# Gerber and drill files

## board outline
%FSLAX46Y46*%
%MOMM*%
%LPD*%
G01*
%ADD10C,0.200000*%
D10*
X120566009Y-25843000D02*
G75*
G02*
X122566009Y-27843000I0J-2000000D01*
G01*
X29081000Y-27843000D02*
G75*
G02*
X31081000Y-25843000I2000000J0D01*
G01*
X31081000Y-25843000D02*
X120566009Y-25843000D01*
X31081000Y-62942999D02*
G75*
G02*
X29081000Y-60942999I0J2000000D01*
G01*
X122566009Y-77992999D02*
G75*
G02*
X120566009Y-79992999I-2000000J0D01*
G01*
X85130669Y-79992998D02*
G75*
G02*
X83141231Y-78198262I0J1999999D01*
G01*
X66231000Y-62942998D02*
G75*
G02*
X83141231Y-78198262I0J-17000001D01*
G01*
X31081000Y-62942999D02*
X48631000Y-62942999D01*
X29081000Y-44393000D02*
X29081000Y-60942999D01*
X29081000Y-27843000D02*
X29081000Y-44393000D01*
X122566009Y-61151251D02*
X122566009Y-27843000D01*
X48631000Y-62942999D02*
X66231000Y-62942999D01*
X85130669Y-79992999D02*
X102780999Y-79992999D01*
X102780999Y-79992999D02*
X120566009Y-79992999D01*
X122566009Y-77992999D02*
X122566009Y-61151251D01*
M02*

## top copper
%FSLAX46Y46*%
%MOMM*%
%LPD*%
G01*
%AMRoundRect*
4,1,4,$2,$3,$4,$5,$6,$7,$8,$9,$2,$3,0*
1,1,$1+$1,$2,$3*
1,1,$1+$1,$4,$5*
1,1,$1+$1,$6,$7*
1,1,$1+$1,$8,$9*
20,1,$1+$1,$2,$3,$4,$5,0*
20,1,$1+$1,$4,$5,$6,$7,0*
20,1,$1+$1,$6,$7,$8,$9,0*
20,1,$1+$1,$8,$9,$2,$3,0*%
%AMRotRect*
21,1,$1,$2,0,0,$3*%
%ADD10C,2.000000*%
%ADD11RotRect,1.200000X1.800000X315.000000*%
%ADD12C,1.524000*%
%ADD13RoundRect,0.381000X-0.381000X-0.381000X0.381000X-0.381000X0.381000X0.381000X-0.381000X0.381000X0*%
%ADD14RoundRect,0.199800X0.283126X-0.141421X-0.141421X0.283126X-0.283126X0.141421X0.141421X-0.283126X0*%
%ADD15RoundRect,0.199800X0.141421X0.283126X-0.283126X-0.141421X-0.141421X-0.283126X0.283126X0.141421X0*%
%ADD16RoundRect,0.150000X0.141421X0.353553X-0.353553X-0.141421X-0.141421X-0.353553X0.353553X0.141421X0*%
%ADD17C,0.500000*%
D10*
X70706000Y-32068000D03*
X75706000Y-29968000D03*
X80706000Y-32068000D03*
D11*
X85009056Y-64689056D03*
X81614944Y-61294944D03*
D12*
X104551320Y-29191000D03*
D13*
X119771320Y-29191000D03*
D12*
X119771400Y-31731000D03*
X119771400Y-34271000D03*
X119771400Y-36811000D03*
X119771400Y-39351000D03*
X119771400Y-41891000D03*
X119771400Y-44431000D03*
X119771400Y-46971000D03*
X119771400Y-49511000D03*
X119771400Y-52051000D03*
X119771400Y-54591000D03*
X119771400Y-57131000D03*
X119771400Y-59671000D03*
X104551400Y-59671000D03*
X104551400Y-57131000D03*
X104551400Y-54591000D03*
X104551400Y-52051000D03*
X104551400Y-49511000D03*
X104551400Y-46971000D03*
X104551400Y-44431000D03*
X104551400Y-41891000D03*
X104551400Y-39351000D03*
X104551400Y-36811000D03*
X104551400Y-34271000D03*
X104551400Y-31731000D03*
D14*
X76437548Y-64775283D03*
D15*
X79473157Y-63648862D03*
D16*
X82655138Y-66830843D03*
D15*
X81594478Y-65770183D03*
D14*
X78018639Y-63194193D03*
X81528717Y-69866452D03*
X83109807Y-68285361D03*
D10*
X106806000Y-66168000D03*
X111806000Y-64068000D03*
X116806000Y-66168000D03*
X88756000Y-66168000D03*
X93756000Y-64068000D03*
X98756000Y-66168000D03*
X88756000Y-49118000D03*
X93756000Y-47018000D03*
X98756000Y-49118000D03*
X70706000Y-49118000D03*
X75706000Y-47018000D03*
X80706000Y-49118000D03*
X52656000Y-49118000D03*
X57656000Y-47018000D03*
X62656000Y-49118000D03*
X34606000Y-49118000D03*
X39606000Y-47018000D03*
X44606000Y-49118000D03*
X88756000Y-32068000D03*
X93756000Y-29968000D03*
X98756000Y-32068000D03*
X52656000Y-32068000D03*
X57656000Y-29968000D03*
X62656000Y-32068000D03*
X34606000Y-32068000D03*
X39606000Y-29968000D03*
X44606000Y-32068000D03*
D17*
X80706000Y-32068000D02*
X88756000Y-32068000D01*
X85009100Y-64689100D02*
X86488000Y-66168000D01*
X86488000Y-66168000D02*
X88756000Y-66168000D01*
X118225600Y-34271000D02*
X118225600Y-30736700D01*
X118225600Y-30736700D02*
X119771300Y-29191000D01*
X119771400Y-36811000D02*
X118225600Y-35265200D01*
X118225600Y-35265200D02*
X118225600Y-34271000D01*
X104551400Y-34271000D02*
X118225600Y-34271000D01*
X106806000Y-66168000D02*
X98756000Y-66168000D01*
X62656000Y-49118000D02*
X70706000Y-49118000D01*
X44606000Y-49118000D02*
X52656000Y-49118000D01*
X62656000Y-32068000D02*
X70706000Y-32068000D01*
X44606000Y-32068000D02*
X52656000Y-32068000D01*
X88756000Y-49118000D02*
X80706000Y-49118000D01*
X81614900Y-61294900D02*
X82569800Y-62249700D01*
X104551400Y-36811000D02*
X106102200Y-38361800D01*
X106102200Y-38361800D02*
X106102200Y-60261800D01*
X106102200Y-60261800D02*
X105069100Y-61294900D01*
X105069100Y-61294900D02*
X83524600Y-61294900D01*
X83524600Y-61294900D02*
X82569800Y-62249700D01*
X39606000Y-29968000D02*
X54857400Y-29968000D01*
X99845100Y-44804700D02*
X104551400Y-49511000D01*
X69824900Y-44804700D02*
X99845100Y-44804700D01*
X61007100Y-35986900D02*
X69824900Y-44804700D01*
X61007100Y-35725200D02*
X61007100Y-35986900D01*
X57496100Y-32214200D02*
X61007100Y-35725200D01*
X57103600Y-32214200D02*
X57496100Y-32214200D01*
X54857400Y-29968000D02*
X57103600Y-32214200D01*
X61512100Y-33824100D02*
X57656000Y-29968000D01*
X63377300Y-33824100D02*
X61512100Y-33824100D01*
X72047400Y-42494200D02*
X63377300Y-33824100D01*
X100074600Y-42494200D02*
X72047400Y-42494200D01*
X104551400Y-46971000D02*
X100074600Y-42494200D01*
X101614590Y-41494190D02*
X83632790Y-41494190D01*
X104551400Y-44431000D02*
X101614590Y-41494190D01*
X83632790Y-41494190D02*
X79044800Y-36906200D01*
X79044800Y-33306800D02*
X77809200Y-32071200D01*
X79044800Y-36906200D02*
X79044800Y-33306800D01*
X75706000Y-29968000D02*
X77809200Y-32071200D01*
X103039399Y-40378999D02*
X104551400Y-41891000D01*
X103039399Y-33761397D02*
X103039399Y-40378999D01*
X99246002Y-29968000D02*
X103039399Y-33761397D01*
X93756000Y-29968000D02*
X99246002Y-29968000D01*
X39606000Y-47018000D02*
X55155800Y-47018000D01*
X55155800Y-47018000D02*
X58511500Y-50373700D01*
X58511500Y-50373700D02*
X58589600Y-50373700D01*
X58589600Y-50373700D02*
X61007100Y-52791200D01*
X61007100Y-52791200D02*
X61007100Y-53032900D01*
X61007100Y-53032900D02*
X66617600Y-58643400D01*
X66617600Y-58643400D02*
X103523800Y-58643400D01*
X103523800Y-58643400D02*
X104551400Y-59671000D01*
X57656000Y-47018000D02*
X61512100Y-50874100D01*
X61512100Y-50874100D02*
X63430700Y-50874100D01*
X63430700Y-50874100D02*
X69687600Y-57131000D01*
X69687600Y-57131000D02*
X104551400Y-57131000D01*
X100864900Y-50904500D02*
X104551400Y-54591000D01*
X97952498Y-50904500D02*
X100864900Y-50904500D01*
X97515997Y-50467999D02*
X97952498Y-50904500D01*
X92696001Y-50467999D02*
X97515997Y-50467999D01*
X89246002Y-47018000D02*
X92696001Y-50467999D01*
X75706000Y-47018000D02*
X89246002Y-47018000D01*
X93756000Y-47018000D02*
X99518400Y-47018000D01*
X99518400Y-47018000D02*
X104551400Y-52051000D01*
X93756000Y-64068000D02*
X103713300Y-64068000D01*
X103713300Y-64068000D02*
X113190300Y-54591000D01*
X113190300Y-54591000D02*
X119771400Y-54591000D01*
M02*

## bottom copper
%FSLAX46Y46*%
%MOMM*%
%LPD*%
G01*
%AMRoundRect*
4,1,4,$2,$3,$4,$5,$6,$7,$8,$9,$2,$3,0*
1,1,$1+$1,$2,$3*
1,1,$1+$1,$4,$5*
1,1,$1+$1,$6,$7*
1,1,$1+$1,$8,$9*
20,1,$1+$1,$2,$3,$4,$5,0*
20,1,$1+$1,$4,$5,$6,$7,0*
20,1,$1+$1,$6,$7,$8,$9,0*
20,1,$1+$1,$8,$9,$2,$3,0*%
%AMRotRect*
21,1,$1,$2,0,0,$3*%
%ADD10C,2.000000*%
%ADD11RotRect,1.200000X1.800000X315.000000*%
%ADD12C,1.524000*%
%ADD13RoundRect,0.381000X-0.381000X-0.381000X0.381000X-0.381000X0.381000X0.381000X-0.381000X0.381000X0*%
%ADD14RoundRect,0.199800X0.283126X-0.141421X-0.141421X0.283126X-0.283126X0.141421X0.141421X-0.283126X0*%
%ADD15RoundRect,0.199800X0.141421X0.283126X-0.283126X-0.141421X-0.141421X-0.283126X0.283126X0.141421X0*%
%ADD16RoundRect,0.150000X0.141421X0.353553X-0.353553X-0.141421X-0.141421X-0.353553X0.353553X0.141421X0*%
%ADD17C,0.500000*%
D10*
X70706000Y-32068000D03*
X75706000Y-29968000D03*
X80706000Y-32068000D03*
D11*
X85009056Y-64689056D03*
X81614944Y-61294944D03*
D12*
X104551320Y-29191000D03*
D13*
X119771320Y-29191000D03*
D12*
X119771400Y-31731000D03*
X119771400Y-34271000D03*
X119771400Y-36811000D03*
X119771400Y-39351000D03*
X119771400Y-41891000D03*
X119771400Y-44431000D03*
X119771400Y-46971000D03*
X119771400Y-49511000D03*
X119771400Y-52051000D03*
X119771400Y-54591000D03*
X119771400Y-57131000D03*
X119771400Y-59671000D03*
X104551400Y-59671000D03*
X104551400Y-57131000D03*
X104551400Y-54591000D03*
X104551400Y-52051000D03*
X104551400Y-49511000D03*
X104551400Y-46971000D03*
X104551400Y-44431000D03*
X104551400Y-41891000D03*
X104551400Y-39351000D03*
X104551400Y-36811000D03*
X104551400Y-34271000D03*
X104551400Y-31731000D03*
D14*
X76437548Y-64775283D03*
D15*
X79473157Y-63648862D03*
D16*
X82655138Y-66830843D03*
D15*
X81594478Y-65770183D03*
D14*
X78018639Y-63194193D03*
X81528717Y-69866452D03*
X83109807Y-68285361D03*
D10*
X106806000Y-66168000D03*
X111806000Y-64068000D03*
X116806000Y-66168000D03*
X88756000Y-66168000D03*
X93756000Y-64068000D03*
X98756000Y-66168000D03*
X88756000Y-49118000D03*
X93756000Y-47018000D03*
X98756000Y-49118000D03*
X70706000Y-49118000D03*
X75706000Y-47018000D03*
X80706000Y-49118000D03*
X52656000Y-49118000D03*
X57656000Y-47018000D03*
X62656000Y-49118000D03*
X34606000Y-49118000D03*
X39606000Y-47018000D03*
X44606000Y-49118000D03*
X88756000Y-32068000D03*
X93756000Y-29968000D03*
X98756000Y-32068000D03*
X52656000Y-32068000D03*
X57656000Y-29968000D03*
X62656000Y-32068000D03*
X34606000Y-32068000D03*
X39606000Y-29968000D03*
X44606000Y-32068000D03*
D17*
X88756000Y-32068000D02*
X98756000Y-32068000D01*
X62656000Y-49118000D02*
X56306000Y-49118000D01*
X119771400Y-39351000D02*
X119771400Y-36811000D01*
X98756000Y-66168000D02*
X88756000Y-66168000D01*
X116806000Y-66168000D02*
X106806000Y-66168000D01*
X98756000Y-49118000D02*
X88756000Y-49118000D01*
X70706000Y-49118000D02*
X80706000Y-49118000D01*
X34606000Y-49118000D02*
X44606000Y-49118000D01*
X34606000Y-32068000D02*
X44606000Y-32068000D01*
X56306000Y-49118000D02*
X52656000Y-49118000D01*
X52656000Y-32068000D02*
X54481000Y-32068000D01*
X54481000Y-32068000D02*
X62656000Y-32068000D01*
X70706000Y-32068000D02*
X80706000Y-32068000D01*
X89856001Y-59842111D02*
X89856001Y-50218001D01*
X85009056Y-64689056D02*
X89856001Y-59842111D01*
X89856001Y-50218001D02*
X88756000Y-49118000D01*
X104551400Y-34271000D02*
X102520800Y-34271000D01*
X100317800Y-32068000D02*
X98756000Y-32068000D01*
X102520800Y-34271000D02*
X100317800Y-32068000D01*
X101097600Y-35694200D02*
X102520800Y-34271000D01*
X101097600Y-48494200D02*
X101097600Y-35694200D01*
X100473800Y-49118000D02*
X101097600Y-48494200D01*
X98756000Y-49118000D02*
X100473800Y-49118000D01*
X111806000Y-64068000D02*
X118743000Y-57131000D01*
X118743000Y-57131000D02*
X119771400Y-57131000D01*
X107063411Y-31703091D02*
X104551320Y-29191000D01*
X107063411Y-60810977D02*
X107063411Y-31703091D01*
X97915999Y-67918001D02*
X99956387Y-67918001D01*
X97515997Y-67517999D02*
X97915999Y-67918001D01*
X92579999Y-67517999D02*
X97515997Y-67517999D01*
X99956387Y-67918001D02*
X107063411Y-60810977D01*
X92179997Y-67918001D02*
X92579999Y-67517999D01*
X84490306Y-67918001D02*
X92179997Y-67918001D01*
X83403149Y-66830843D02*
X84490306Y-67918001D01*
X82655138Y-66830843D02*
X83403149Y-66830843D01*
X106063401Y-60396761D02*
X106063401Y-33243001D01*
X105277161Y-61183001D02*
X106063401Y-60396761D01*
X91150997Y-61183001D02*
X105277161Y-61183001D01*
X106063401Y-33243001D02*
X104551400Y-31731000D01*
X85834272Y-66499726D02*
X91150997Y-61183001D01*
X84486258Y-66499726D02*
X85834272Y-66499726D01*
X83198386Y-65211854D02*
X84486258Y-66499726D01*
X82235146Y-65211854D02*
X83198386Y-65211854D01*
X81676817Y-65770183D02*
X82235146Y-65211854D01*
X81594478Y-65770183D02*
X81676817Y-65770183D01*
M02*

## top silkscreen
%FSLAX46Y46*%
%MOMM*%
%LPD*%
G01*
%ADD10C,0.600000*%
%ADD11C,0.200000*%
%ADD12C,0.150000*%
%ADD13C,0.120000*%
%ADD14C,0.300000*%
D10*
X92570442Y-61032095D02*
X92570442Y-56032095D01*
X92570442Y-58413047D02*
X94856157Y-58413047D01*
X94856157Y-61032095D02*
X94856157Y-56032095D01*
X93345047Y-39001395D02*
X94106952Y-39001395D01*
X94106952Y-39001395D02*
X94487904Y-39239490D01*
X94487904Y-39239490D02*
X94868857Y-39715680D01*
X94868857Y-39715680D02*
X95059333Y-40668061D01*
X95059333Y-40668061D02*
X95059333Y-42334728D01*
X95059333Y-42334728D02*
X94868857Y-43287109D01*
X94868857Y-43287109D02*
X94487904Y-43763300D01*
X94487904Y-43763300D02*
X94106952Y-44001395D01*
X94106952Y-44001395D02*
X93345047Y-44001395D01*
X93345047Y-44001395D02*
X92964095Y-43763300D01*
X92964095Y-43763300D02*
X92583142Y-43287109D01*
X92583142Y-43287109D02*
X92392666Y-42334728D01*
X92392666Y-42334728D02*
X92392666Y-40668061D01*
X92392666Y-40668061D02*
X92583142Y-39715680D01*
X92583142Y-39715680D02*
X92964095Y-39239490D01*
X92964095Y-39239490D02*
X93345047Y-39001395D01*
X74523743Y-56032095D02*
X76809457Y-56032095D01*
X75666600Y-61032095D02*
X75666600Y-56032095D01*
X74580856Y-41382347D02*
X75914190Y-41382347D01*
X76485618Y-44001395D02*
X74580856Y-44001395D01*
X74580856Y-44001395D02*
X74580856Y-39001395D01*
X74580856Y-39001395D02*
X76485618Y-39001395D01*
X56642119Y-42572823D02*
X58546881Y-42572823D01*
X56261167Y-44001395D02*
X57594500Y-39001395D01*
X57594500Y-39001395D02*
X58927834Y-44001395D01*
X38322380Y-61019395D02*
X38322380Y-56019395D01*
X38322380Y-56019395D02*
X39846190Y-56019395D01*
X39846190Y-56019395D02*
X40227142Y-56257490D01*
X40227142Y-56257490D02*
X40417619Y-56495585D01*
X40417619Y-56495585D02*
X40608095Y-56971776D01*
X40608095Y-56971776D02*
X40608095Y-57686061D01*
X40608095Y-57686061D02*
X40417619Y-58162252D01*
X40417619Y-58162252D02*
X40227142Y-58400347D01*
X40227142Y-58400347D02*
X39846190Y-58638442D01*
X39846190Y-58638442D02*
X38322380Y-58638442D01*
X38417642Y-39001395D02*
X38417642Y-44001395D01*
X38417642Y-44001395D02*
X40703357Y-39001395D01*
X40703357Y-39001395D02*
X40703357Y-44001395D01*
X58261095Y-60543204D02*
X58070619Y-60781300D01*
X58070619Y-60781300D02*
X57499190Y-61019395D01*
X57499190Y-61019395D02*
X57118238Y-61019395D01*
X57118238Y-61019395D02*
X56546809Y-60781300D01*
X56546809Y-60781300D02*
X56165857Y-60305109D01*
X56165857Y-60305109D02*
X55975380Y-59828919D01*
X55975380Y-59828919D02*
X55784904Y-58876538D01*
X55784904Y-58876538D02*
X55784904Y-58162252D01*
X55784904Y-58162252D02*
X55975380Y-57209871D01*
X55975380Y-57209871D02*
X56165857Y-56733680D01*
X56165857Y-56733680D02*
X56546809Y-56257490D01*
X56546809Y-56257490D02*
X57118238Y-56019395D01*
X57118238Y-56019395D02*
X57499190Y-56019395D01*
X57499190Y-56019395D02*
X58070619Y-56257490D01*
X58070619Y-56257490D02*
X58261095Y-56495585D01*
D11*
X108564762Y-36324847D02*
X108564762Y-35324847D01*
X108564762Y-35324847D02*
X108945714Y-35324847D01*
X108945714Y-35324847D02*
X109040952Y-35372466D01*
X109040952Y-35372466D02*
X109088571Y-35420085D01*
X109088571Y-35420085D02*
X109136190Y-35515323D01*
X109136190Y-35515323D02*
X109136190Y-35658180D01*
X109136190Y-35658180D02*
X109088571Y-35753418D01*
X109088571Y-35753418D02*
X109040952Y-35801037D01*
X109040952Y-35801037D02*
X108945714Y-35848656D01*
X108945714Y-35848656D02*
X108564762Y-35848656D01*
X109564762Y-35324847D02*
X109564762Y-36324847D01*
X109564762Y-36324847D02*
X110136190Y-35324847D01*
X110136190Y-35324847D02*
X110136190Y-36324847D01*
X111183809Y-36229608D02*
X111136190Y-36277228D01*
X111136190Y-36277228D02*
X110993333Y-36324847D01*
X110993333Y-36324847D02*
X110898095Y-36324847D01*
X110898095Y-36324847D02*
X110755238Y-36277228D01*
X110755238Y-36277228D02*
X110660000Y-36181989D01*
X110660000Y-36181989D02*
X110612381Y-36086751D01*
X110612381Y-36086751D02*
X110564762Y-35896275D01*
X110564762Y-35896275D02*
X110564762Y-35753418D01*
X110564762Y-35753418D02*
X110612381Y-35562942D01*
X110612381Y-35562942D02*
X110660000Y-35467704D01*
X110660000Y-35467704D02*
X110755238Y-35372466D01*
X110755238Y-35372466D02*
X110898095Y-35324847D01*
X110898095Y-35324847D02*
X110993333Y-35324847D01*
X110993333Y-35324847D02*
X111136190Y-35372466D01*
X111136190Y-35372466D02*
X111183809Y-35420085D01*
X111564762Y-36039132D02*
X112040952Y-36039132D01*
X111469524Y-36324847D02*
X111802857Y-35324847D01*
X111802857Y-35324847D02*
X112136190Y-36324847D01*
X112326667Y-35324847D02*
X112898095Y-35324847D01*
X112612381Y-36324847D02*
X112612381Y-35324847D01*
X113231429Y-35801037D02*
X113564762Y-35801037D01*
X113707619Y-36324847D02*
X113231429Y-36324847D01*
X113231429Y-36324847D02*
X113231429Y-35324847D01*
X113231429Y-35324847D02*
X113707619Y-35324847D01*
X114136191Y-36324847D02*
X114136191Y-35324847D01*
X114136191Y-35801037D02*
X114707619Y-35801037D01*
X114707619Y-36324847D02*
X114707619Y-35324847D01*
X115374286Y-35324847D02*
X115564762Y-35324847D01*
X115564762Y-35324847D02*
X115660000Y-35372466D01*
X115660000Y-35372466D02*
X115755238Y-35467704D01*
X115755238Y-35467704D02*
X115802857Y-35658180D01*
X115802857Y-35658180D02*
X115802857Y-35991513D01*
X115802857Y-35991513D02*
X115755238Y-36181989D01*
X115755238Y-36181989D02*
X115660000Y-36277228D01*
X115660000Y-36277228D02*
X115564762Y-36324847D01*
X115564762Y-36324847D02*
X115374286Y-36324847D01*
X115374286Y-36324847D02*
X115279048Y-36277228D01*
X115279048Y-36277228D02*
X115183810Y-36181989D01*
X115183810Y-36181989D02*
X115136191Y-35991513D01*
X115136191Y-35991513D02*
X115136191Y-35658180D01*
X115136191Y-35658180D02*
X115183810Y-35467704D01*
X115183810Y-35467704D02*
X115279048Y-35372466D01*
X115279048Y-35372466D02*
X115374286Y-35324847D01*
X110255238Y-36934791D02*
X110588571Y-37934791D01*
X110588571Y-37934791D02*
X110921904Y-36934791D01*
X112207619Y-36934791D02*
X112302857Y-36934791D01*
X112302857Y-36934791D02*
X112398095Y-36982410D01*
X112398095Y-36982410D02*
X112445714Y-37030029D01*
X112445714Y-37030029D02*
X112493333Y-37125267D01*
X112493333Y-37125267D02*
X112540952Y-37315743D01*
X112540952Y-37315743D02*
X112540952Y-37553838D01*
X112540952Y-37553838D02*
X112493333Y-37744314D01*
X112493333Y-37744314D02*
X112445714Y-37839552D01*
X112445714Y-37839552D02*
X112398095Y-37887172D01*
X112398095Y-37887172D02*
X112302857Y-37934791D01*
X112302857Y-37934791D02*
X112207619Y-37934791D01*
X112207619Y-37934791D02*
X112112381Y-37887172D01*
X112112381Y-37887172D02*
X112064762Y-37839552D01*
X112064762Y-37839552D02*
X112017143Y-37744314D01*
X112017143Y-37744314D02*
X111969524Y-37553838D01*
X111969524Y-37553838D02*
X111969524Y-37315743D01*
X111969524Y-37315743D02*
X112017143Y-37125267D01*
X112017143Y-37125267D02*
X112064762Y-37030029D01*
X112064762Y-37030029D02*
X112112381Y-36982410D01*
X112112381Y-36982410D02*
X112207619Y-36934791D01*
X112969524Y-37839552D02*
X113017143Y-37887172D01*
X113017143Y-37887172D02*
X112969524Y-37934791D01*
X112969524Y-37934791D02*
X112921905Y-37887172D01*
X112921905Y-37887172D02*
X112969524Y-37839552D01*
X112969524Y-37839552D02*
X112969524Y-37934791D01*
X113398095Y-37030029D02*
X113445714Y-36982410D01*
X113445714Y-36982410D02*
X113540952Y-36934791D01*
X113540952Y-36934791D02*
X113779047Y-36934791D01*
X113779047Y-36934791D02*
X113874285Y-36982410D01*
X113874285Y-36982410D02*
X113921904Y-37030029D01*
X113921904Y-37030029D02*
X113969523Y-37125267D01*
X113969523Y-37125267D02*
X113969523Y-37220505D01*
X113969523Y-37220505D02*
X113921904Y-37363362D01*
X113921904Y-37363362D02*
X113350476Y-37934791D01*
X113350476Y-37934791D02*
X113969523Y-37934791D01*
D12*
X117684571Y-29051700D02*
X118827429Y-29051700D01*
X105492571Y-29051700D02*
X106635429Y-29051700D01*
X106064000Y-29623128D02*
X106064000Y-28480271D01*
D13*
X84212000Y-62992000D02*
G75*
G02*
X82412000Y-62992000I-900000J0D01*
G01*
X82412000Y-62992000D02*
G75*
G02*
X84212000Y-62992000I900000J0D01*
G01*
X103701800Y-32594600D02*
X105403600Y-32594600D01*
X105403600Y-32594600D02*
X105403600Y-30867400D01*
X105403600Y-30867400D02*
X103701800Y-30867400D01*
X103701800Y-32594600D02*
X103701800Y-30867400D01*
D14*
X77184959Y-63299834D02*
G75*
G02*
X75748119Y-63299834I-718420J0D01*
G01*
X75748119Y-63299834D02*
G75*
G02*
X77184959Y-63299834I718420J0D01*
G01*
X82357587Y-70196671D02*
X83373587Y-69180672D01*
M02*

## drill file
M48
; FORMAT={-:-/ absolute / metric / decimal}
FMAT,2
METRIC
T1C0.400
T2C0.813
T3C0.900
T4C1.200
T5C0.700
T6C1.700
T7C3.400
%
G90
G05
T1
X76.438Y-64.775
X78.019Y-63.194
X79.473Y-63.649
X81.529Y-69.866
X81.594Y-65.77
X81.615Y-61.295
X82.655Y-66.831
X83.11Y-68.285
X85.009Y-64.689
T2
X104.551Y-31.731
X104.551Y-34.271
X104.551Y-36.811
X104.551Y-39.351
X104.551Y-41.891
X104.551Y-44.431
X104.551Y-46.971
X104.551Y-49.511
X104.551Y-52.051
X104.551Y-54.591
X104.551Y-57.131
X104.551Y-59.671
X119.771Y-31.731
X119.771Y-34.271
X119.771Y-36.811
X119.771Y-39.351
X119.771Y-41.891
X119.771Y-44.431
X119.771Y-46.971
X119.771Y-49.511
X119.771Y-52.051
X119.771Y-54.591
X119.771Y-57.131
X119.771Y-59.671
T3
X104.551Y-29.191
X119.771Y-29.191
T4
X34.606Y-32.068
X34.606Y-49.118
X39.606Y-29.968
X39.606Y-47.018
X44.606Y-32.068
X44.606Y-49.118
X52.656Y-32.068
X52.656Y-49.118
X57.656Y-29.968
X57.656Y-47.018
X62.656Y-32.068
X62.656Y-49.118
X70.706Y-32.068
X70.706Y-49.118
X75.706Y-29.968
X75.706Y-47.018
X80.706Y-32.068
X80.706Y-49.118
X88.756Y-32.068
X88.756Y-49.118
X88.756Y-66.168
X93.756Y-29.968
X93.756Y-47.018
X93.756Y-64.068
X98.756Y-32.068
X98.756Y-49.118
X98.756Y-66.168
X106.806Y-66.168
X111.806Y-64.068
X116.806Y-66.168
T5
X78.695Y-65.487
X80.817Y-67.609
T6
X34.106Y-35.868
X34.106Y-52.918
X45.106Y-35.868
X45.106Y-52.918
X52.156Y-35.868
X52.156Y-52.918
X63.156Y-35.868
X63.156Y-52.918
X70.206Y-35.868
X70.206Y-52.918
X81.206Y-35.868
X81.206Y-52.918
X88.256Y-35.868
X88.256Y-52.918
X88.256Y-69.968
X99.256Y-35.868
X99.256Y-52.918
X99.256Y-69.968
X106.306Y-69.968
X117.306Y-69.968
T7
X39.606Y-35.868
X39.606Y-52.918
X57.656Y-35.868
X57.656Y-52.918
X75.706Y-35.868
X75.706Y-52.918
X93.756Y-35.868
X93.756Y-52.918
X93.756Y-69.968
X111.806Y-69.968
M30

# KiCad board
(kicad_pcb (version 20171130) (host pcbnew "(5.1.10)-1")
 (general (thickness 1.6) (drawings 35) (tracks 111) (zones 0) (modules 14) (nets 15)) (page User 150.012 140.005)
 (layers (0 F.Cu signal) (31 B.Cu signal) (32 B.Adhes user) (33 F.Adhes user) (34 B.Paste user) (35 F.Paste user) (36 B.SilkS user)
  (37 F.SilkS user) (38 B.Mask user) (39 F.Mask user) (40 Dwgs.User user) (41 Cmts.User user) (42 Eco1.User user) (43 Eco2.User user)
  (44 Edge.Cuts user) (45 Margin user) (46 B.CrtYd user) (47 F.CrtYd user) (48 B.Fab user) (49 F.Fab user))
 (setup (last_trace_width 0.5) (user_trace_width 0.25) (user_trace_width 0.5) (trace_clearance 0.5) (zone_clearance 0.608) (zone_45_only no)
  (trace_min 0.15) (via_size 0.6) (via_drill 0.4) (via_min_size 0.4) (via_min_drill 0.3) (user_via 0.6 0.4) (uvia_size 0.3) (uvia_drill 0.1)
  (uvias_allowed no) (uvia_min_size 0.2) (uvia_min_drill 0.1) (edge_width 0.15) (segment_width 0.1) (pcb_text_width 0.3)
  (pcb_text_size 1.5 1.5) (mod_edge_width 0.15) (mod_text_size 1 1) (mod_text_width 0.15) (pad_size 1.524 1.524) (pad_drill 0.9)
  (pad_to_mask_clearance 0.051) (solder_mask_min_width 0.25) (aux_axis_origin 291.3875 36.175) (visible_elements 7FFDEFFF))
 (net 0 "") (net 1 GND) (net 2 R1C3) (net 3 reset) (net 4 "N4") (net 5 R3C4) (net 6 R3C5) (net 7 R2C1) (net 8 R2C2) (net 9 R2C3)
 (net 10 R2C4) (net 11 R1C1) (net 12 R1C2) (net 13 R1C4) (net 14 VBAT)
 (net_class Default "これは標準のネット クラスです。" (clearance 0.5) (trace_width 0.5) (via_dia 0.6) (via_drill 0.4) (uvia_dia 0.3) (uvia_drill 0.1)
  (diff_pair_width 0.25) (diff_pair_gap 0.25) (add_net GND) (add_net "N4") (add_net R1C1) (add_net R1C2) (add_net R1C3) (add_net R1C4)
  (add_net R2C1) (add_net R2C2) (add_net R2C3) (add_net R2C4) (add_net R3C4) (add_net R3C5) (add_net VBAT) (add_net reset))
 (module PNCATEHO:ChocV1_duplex (layer F.Cu) (at 75.706 35.868)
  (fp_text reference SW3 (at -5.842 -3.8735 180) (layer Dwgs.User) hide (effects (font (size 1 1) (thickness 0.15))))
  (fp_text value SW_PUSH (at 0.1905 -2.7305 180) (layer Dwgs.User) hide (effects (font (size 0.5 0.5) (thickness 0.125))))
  (pad 2 thru_hole circle (at -5 -3.8) (size 2 2) (drill 1.2) (layers *.Cu *.Mask) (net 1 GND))
  (pad 1 thru_hole circle (at 0 -5.9) (size 2 2) (drill 1.2) (layers *.Cu *.Mask) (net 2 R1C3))
  (pad "" np_thru_hole circle (at 5.5 0 90) (size 1.7 1.7) (drill 1.7) (layers *.Cu *.Mask))
  (pad "" np_thru_hole circle (at -5.5 0 90) (size 1.7 1.7) (drill 1.7) (layers *.Cu *.Mask))
  (pad "" np_thru_hole circle (at 0 0 90) (size 3.4 3.4) (drill 3.4) (layers *.Cu *.Mask))
  (pad 2 thru_hole circle (at 5 -3.8) (size 2 2) (drill 1.2) (layers *.Cu *.Mask) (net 1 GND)))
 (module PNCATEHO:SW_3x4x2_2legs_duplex (layer F.Cu) (at 83.312 62.992 315)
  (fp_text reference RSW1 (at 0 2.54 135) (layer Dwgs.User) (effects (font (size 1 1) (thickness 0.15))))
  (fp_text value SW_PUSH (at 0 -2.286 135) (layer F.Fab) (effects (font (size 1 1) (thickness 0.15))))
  (fp_circle (center 0 0) (end 0.9 0) (layer F.SilkS) (width 0.12))
  (pad 2 thru_hole rect (at 2.4 0 315) (size 1.2 1.8) (drill 0.4) (layers *.Cu *.Mask) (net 1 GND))
  (pad 1 thru_hole rect (at -2.4 0 315) (size 1.2 1.8) (drill 0.4) (layers *.Cu *.Mask) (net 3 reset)))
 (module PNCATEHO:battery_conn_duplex (layer F.Cu) (at 112.16 28.937)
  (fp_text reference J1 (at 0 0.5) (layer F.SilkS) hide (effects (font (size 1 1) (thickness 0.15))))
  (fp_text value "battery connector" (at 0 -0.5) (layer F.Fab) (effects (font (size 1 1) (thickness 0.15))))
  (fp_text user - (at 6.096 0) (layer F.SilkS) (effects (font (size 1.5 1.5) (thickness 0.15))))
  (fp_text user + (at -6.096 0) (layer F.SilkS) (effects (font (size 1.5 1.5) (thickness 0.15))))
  (pad 1 thru_hole circle (at -7.60868 0.254 90) (size 1.524 1.524) (drill 0.9) (layers *.Cu *.Mask) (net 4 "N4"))
  (pad 2 thru_hole roundrect (at 7.61132 0.254) (size 1.524 1.524) (drill 0.9) (layers *.Cu *.Mask) (roundrect_rratio 0.25) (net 1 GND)))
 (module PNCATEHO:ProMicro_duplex (layer F.Cu) (at 112.16 46.209)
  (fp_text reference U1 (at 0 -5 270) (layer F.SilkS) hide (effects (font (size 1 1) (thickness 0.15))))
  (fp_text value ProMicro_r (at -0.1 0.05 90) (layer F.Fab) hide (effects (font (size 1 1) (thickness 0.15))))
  (fp_line (start -8.4582 -13.6144) (end -6.7564 -13.6144) (layer F.SilkS) (width 0.12))
  (fp_line (start -6.7564 -13.6144) (end -6.7564 -15.3416) (layer F.SilkS) (width 0.12))
  (fp_line (start -6.7564 -15.3416) (end -8.4582 -15.3416) (layer F.SilkS) (width 0.12))
  (fp_line (start -8.4582 -13.6144) (end -8.4582 -15.3416) (layer F.SilkS) (width 0.12))
  (pad 1 thru_hole circle (at 7.6114 -14.478) (size 1.524 1.524) (drill 0.8128) (layers *.Cu *.Mask))
  (pad 2 thru_hole circle (at 7.6114 -11.938) (size 1.524 1.524) (drill 0.8128) (layers *.Cu *.Mask))
  (pad 3 thru_hole circle (at 7.6114 -9.398) (size 1.524 1.524) (drill 0.8128) (layers *.Cu *.Mask) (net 1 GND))
  (pad 4 thru_hole circle (at 7.6114 -6.858) (size 1.524 1.524) (drill 0.8128) (layers *.Cu *.Mask) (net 1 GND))
  (pad 5 thru_hole circle (at 7.6114 -4.318) (size 1.524 1.524) (drill 0.8128) (layers *.Cu *.Mask))
  (pad 6 thru_hole circle (at 7.6114 -1.778) (size 1.524 1.524) (drill 0.8128) (layers *.Cu *.Mask))
  (pad 7 thru_hole circle (at 7.6114 0.762) (size 1.524 1.524) (drill 0.8128) (layers *.Cu *.Mask))
  (pad 8 thru_hole circle (at 7.6114 3.302) (size 1.524 1.524) (drill 0.8128) (layers *.Cu *.Mask))
  (pad 9 thru_hole circle (at 7.6114 5.842) (size 1.524 1.524) (drill 0.8128) (layers *.Cu *.Mask))
  (pad 10 thru_hole circle (at 7.6114 8.382) (size 1.524 1.524) (drill 0.8128) (layers *.Cu *.Mask) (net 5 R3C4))
  (pad 11 thru_hole circle (at 7.6114 10.922) (size 1.524 1.524) (drill 0.8128) (layers *.Cu *.Mask) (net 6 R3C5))
  (pad 12 thru_hole circle (at 7.6114 13.462) (size 1.524 1.524) (drill 0.8128) (layers *.Cu *.Mask))
  (pad 13 thru_hole circle (at -7.6086 13.462) (size 1.524 1.524) (drill 0.8128) (layers *.Cu *.Mask) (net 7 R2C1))
  (pad 14 thru_hole circle (at -7.6086 10.922) (size 1.524 1.524) (drill 0.8128) (layers *.Cu *.Mask) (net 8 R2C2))
  (pad 15 thru_hole circle (at -7.6086 8.382) (size 1.524 1.524) (drill 0.8128) (layers *.Cu *.Mask) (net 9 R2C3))
  (pad 16 thru_hole circle (at -7.6086 5.842) (size 1.524 1.524) (drill 0.8128) (layers *.Cu *.Mask) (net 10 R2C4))
  (pad 17 thru_hole circle (at -7.6086 3.302) (size 1.524 1.524) (drill 0.8128) (layers *.Cu *.Mask) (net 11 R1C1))
  (pad 18 thru_hole circle (at -7.6086 0.762) (size 1.524 1.524) (drill 0.8128) (layers *.Cu *.Mask) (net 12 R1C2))
  (pad 19 thru_hole circle (at -7.6086 -1.778) (size 1.524 1.524) (drill 0.8128) (layers *.Cu *.Mask) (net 2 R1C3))
  (pad 20 thru_hole circle (at -7.6086 -4.318) (size 1.524 1.524) (drill 0.8128) (layers *.Cu *.Mask) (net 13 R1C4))
  (pad 21 thru_hole circle (at -7.6086 -6.858) (size 1.524 1.524) (drill 0.8128) (layers *.Cu *.Mask))
  (pad 22 thru_hole circle (at -7.6086 -9.398) (size 1.524 1.524) (drill 0.8128) (layers *.Cu *.Mask) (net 3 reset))
  (pad 23 thru_hole circle (at -7.6086 -11.938) (size 1.524 1.524) (drill 0.8128) (layers *.Cu *.Mask) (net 1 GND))
  (pad 24 thru_hole circle (at -7.6086 -14.478 90) (size 1.524 1.524) (drill 0.8128) (layers *.Cu *.Mask) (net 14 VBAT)))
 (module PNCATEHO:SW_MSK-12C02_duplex (layer F.Cu) (at 79.756 66.548 135)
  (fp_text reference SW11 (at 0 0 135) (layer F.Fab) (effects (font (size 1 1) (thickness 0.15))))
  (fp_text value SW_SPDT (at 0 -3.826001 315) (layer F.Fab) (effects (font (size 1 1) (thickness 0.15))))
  (fp_circle (center 4.6228 -0.0292) (end 4.6228 0.68922) (layer F.SilkS) (width 0.3))
  (fp_line (start -4.4196 -0.7404) (end -4.4196 0.69644) (layer F.SilkS) (width 0.3))
  (pad "" thru_hole roundrect (at 3.6 -1.093 135) (size 1 0.6) (drill 0.4) (layers *.Cu *.Mask) (roundrect_rratio 0.333))
  (pad 1 thru_hole roundrect (at 2.25 1.85 225) (size 1 0.6) (drill 0.4) (layers *.Cu *.Mask) (roundrect_rratio 0.333))
  (pad 3 thru_hole roundrect (at -2.25 1.85 225) (size 1 0.6) (drill 0.4) (layers *.Cu *.Mask) (roundrect_rratio 0.25) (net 4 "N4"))
  (pad 2 thru_hole roundrect (at -0.75 1.85 225) (size 1 0.6) (drill 0.4) (layers *.Cu *.Mask) (roundrect_rratio 0.333) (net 14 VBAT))
  (pad "" np_thru_hole circle (at -1.5 0 225) (size 0.7 0.7) (drill 0.7) (layers *.Cu *.Mask))
  (pad "" np_thru_hole circle (at 1.5 0 225) (size 0.7 0.7) (drill 0.7) (layers *.Cu *.Mask))
  (pad "" thru_hole roundrect (at 3.6 1.143 135) (size 1 0.6) (drill 0.4) (layers *.Cu *.Mask) (roundrect_rratio 0.333))
  (pad "" thru_hole roundrect (at -3.6 -1.093 135) (size 1 0.6) (drill 0.4) (layers *.Cu *.Mask) (roundrect_rratio 0.333))
  (pad "" thru_hole roundrect (at -3.6 1.143 135) (size 1 0.6) (drill 0.4) (layers *.Cu *.Mask) (roundrect_rratio 0.333)))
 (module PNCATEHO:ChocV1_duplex (layer F.Cu) (at 111.806 69.968)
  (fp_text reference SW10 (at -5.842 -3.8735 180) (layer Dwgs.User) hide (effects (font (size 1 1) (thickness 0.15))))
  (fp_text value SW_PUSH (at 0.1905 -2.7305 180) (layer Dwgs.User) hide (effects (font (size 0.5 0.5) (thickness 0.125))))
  (pad 2 thru_hole circle (at -5 -3.8) (size 2 2) (drill 1.2) (layers *.Cu *.Mask) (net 1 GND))
  (pad 1 thru_hole circle (at 0 -5.9) (size 2 2) (drill 1.2) (layers *.Cu *.Mask) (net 6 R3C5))
  (pad "" np_thru_hole circle (at 5.5 0 90) (size 1.7 1.7) (drill 1.7) (layers *.Cu *.Mask))
  (pad "" np_thru_hole circle (at -5.5 0 90) (size 1.7 1.7) (drill 1.7) (layers *.Cu *.Mask))
  (pad "" np_thru_hole circle (at 0 0 90) (size 3.4 3.4) (drill 3.4) (layers *.Cu *.Mask))
  (pad 2 thru_hole circle (at 5 -3.8) (size 2 2) (drill 1.2) (layers *.Cu *.Mask) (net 1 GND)))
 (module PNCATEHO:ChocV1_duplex (layer F.Cu) (at 93.756 69.968)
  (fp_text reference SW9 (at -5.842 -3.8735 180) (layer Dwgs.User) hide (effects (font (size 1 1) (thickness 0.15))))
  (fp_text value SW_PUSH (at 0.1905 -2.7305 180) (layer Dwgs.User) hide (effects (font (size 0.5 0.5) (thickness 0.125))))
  (pad 2 thru_hole circle (at -5 -3.8) (size 2 2) (drill 1.2) (layers *.Cu *.Mask) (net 1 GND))
  (pad 1 thru_hole circle (at 0 -5.9) (size 2 2) (drill 1.2) (layers *.Cu *.Mask) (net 5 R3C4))
  (pad "" np_thru_hole circle (at 5.5 0 90) (size 1.7 1.7) (drill 1.7) (layers *.Cu *.Mask))
  (pad "" np_thru_hole circle (at -5.5 0 90) (size 1.7 1.7) (drill 1.7) (layers *.Cu *.Mask))
  (pad "" np_thru_hole circle (at 0 0 90) (size 3.4 3.4) (drill 3.4) (layers *.Cu *.Mask))
  (pad 2 thru_hole circle (at 5 -3.8) (size 2 2) (drill 1.2) (layers *.Cu *.Mask) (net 1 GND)))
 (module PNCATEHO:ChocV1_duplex (layer F.Cu) (at 93.756 52.918)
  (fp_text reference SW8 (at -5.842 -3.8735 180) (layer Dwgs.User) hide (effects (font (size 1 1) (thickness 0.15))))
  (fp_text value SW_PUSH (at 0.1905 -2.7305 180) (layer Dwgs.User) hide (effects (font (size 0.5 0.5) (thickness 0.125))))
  (pad 2 thru_hole circle (at -5 -3.8) (size 2 2) (drill 1.2) (layers *.Cu *.Mask) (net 1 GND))
  (pad 1 thru_hole circle (at 0 -5.9) (size 2 2) (drill 1.2) (layers *.Cu *.Mask) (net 10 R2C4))
  (pad "" np_thru_hole circle (at 5.5 0 90) (size 1.7 1.7) (drill 1.7) (layers *.Cu *.Mask))
  (pad "" np_thru_hole circle (at -5.5 0 90) (size 1.7 1.7) (drill 1.7) (layers *.Cu *.Mask))
  (pad "" np_thru_hole circle (at 0 0 90) (size 3.4 3.4) (drill 3.4) (layers *.Cu *.Mask))
  (pad 2 thru_hole circle (at 5 -3.8) (size 2 2) (drill 1.2) (layers *.Cu *.Mask) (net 1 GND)))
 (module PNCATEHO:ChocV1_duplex (layer F.Cu) (at 75.706 52.918)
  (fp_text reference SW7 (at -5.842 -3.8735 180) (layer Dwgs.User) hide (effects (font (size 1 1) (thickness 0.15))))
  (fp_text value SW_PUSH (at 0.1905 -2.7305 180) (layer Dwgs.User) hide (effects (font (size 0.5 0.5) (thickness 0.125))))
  (pad 2 thru_hole circle (at -5 -3.8) (size 2 2) (drill 1.2) (layers *.Cu *.Mask) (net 1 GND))
  (pad 1 thru_hole circle (at 0 -5.9) (size 2 2) (drill 1.2) (layers *.Cu *.Mask) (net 9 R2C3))
  (pad "" np_thru_hole circle (at 5.5 0 90) (size 1.7 1.7) (drill 1.7) (layers *.Cu *.Mask))
  (pad "" np_thru_hole circle (at -5.5 0 90) (size 1.7 1.7) (drill 1.7) (layers *.Cu *.Mask))
  (pad "" np_thru_hole circle (at 0 0 90) (size 3.4 3.4) (drill 3.4) (layers *.Cu *.Mask))
  (pad 2 thru_hole circle (at 5 -3.8) (size 2 2) (drill 1.2) (layers *.Cu *.Mask) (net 1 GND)))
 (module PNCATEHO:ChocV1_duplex (layer F.Cu) (at 57.656 52.918)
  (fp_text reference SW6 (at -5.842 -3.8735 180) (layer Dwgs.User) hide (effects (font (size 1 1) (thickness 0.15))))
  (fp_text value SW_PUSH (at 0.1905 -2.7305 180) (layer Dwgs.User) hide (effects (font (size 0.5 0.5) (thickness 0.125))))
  (pad 2 thru_hole circle (at -5 -3.8) (size 2 2) (drill 1.2) (layers *.Cu *.Mask) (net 1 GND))
  (pad 1 thru_hole circle (at 0 -5.9) (size 2 2) (drill 1.2) (layers *.Cu *.Mask) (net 8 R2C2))
  (pad "" np_thru_hole circle (at 5.5 0 90) (size 1.7 1.7) (drill 1.7) (layers *.Cu *.Mask))
  (pad "" np_thru_hole circle (at -5.5 0 90) (size 1.7 1.7) (drill 1.7) (layers *.Cu *.Mask))
  (pad "" np_thru_hole circle (at 0 0 90) (size 3.4 3.4) (drill 3.4) (layers *.Cu *.Mask))
  (pad 2 thru_hole circle (at 5 -3.8) (size 2 2) (drill 1.2) (layers *.Cu *.Mask) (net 1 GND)))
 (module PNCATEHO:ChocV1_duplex (layer F.Cu) (at 39.606 52.918)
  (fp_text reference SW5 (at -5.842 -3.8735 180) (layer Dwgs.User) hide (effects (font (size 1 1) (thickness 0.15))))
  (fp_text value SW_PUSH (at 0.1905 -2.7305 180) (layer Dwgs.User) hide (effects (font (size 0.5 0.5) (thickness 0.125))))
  (pad 2 thru_hole circle (at -5 -3.8) (size 2 2) (drill 1.2) (layers *.Cu *.Mask) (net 1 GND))
  (pad 1 thru_hole circle (at 0 -5.9) (size 2 2) (drill 1.2) (layers *.Cu *.Mask) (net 7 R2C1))
  (pad "" np_thru_hole circle (at 5.5 0 90) (size 1.7 1.7) (drill 1.7) (layers *.Cu *.Mask))
  (pad "" np_thru_hole circle (at -5.5 0 90) (size 1.7 1.7) (drill 1.7) (layers *.Cu *.Mask))
  (pad "" np_thru_hole circle (at 0 0 90) (size 3.4 3.4) (drill 3.4) (layers *.Cu *.Mask))
  (pad 2 thru_hole circle (at 5 -3.8) (size 2 2) (drill 1.2) (layers *.Cu *.Mask) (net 1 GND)))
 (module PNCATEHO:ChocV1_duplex (layer F.Cu) (at 93.756 35.868)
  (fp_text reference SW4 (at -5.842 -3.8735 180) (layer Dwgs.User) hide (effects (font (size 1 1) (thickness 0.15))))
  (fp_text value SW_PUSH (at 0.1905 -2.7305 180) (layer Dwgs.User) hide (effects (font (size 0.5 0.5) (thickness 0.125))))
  (pad 2 thru_hole circle (at -5 -3.8) (size 2 2) (drill 1.2) (layers *.Cu *.Mask) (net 1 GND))
  (pad 1 thru_hole circle (at 0 -5.9) (size 2 2) (drill 1.2) (layers *.Cu *.Mask) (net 13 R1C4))
  (pad "" np_thru_hole circle (at 5.5 0 90) (size 1.7 1.7) (drill 1.7) (layers *.Cu *.Mask))
  (pad "" np_thru_hole circle (at -5.5 0 90) (size 1.7 1.7) (drill 1.7) (layers *.Cu *.Mask))
  (pad "" np_thru_hole circle (at 0 0 90) (size 3.4 3.4) (drill 3.4) (layers *.Cu *.Mask))
  (pad 2 thru_hole circle (at 5 -3.8) (size 2 2) (drill 1.2) (layers *.Cu *.Mask) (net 1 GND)))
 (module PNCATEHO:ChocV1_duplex (layer F.Cu) (at 57.656 35.868)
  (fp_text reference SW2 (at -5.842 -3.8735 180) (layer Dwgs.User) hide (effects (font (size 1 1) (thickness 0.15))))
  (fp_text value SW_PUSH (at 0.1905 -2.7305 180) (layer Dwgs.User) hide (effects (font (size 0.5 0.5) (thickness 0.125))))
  (pad 2 thru_hole circle (at -5 -3.8) (size 2 2) (drill 1.2) (layers *.Cu *.Mask) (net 1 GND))
  (pad 1 thru_hole circle (at 0 -5.9) (size 2 2) (drill 1.2) (layers *.Cu *.Mask) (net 12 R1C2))
  (pad "" np_thru_hole circle (at 5.5 0 90) (size 1.7 1.7) (drill 1.7) (layers *.Cu *.Mask))
  (pad "" np_thru_hole circle (at -5.5 0 90) (size 1.7 1.7) (drill 1.7) (layers *.Cu *.Mask))
  (pad "" np_thru_hole circle (at 0 0 90) (size 3.4 3.4) (drill 3.4) (layers *.Cu *.Mask))
  (pad 2 thru_hole circle (at 5 -3.8) (size 2 2) (drill 1.2) (layers *.Cu *.Mask) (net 1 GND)))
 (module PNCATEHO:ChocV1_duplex (layer F.Cu) (at 39.606 35.868)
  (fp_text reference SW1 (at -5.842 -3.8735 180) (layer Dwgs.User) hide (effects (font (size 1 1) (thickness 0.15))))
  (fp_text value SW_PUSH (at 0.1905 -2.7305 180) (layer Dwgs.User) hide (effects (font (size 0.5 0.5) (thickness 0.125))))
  (pad 2 thru_hole circle (at -5 -3.8) (size 2 2) (drill 1.2) (layers *.Cu *.Mask) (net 1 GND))
  (pad 1 thru_hole circle (at 0 -5.9) (size 2 2) (drill 1.2) (layers *.Cu *.Mask) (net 11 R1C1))
  (pad "" np_thru_hole circle (at 5.5 0 90) (size 1.7 1.7) (drill 1.7) (layers *.Cu *.Mask))
  (pad "" np_thru_hole circle (at -5.5 0 90) (size 1.7 1.7) (drill 1.7) (layers *.Cu *.Mask))
  (pad "" np_thru_hole circle (at 0 0 90) (size 3.4 3.4) (drill 3.4) (layers *.Cu *.Mask))
  (pad 2 thru_hole circle (at 5 -3.8) (size 2 2) (drill 1.2) (layers *.Cu *.Mask) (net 1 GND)))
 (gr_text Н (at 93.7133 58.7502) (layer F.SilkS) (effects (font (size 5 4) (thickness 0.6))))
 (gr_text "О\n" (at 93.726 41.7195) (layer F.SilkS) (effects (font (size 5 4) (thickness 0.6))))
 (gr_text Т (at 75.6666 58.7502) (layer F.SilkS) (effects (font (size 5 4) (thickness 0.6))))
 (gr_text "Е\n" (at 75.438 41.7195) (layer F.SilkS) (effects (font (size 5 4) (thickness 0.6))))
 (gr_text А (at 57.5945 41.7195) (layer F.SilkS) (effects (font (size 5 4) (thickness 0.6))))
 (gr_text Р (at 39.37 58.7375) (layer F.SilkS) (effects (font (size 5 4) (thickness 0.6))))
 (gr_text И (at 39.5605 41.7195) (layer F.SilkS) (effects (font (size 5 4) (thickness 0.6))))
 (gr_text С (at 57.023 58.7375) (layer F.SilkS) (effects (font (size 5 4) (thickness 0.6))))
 (gr_arc (start 120.566009 27.843) (end 122.566009 27.843) (angle -90) (layer Edge.Cuts) (width 0.2))
 (gr_arc (start 31.081 27.843) (end 31.081 25.843) (angle -90) (layer Edge.Cuts) (width 0.2))
 (gr_line (start 31.081 25.843) (end 120.566009 25.843) (layer Edge.Cuts) (width 0.2))
 (gr_arc (start 31.081 60.942999) (end 29.081 60.942999) (angle -90) (layer Edge.Cuts) (width 0.2))
 (gr_arc (start 120.566009 77.992999) (end 120.566009 79.992999) (angle -90) (layer Edge.Cuts) (width 0.2))
 (gr_arc (start 85.130669 77.992999) (end 83.141231 78.198262) (angle -84.10927124) (layer Edge.Cuts) (width 0.2))
 (gr_arc (start 66.231 79.942999) (end 83.141231 78.198262) (angle -84.10927124) (layer Edge.Cuts) (width 0.2))
 (gr_line (start 31.081 62.942999) (end 48.631 62.942999) (layer Edge.Cuts) (width 0.2))
 (gr_line (start 29.081 44.393) (end 29.081 60.942999) (layer Edge.Cuts) (width 0.2))
 (gr_line (start 29.081 27.843) (end 29.081 44.393) (layer Edge.Cuts) (width 0.2))
 (gr_line (start 122.566009 61.151251) (end 122.566009 27.843) (layer Edge.Cuts) (width 0.2))
 (gr_line (start 48.631 62.942999) (end 66.231 62.942999) (layer Edge.Cuts) (width 0.2))
 (gr_line (start 85.130669 79.992999) (end 102.780999 79.992999) (layer Edge.Cuts) (width 0.2))
 (gr_line (start 102.780999 79.992999) (end 120.566009 79.992999) (layer Edge.Cuts) (width 0.2))
 (gr_line (start 122.566009 77.992999) (end 122.566009 61.151251) (layer Edge.Cuts) (width 0.2))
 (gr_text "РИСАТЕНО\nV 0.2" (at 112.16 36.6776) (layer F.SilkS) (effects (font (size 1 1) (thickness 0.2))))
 (segment (start 88.756 32.068) (end 98.756 32.068) (width 0.5) (layer B.Cu) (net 1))
 (segment (start 80.706 32.068) (end 88.756 32.068) (width 0.5) (layer F.Cu) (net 1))
 (segment (start 85.0091 64.6891) (end 86.488 66.168) (width 0.5) (layer F.Cu) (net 1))
 (segment (start 86.488 66.168) (end 88.756 66.168) (width 0.5) (layer F.Cu) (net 1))
 (segment (start 118.2256 34.271) (end 118.2256 30.7367) (width 0.5) (layer F.Cu) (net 1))
 (segment (start 118.2256 30.7367) (end 119.7713 29.191) (width 0.5) (layer F.Cu) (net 1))
 (segment (start 119.7714 36.811) (end 118.2256 35.2652) (width 0.5) (layer F.Cu) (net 1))
 (segment (start 118.2256 35.2652) (end 118.2256 34.271) (width 0.5) (layer F.Cu) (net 1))
 (segment (start 104.5514 34.271) (end 118.2256 34.271) (width 0.5) (layer F.Cu) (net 1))
 (segment (start 62.656 49.118) (end 56.306 49.118) (width 0.5) (layer B.Cu) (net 1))
 (segment (start 119.7714 39.351) (end 119.7714 36.811) (width 0.5) (layer B.Cu) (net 1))
 (segment (start 98.756 66.168) (end 88.756 66.168) (width 0.5) (layer B.Cu) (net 1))
 (segment (start 106.806 66.168) (end 98.756 66.168) (width 0.5) (layer F.Cu) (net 1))
 (segment (start 116.806 66.168) (end 106.806 66.168) (width 0.5) (layer B.Cu) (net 1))
 (segment (start 98.756 49.118) (end 88.756 49.118) (width 0.5) (layer B.Cu) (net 1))
 (segment (start 70.706 49.118) (end 80.706 49.118) (width 0.5) (layer B.Cu) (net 1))
 (segment (start 62.656 49.118) (end 70.706 49.118) (width 0.5) (layer F.Cu) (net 1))
 (segment (start 34.606 49.118) (end 44.606 49.118) (width 0.5) (layer B.Cu) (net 1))
 (segment (start 44.606 49.118) (end 52.656 49.118) (width 0.5) (layer F.Cu) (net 1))
 (segment (start 62.656 32.068) (end 70.706 32.068) (width 0.5) (layer F.Cu) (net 1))
 (segment (start 34.606 32.068) (end 44.606 32.068) (width 0.5) (layer B.Cu) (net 1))
 (segment (start 44.606 32.068) (end 52.656 32.068) (width 0.5) (layer F.Cu) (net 1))
 (segment (start 88.756 49.118) (end 80.706 49.118) (width 0.5) (layer F.Cu) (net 1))
 (segment (start 56.306 49.118) (end 52.656 49.118) (width 0.5) (layer B.Cu) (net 1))
 (segment (start 52.656 32.068) (end 54.481 32.068) (width 0.5) (layer B.Cu) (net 1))
 (segment (start 54.481 32.068) (end 62.656 32.068) (width 0.5) (layer B.Cu) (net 1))
 (segment (start 70.706 32.068) (end 80.706 32.068) (width 0.5) (layer B.Cu) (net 1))
 (segment (start 89.856001 59.842111) (end 89.856001 50.218001) (width 0.5) (layer B.Cu) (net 1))
 (segment (start 85.009056 64.689056) (end 89.856001 59.842111) (width 0.5) (layer B.Cu) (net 1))
 (segment (start 89.856001 50.218001) (end 88.756 49.118) (width 0.5) (layer B.Cu) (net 1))
 (segment (start 104.5514 34.271) (end 102.5208 34.271) (width 0.5) (layer B.Cu) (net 1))
 (segment (start 100.3178 32.068) (end 98.756 32.068) (width 0.5) (layer B.Cu) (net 1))
 (segment (start 102.5208 34.271) (end 100.3178 32.068) (width 0.5) (layer B.Cu) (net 1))
 (segment (start 101.0976 35.6942) (end 102.5208 34.271) (width 0.5) (layer B.Cu) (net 1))
 (segment (start 101.0976 48.4942) (end 101.0976 35.6942) (width 0.5) (layer B.Cu) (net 1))
 (segment (start 100.4738 49.118) (end 101.0976 48.4942) (width 0.5) (layer B.Cu) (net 1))
 (segment (start 98.756 49.118) (end 100.4738 49.118) (width 0.5) (layer B.Cu) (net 1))
 (segment (start 81.6149 61.2949) (end 82.5698 62.2497) (width 0.5) (layer F.Cu) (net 3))
 (segment (start 104.5514 36.811) (end 106.1022 38.3618) (width 0.5) (layer F.Cu) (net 3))
 (segment (start 106.1022 38.3618) (end 106.1022 60.2618) (width 0.5) (layer F.Cu) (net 3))
 (segment (start 106.1022 60.2618) (end 105.0691 61.2949) (width 0.5) (layer F.Cu) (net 3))
 (segment (start 105.0691 61.2949) (end 83.5246 61.2949) (width 0.5) (layer F.Cu) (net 3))
 (segment (start 83.5246 61.2949) (end 82.5698 62.2497) (width 0.5) (layer F.Cu) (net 3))
 (segment (start 39.606 29.968) (end 54.8574 29.968) (width 0.5) (layer F.Cu) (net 11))
 (segment (start 99.8451 44.8047) (end 104.5514 49.511) (width 0.5) (layer F.Cu) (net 11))
 (segment (start 69.8249 44.8047) (end 99.8451 44.8047) (width 0.5) (layer F.Cu) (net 11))
 (segment (start 61.0071 35.9869) (end 69.8249 44.8047) (width 0.5) (layer F.Cu) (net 11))
 (segment (start 61.0071 35.7252) (end 61.0071 35.9869) (width 0.5) (layer F.Cu) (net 11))
 (segment (start 57.4961 32.2142) (end 61.0071 35.7252) (width 0.5) (layer F.Cu) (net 11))
 (segment (start 57.1036 32.2142) (end 57.4961 32.2142) (width 0.5) (layer F.Cu) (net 11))
 (segment (start 54.8574 29.968) (end 57.1036 32.2142) (width 0.5) (layer F.Cu) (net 11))
 (segment (start 61.5121 33.8241) (end 57.656 29.968) (width 0.5) (layer F.Cu) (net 12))
 (segment (start 63.3773 33.8241) (end 61.5121 33.8241) (width 0.5) (layer F.Cu) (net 12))
 (segment (start 72.0474 42.4942) (end 63.3773 33.8241) (width 0.5) (layer F.Cu) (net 12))
 (segment (start 100.0746 42.4942) (end 72.0474 42.4942) (width 0.5) (layer F.Cu) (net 12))
 (segment (start 104.5514 46.971) (end 100.0746 42.4942) (width 0.5) (layer F.Cu) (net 12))
 (segment (start 101.61459 41.49419) (end 83.63279 41.49419) (width 0.5) (layer F.Cu) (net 2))
 (segment (start 104.5514 44.431) (end 101.61459 41.49419) (width 0.5) (layer F.Cu) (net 2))
 (segment (start 83.63279 41.49419) (end 79.0448 36.9062) (width 0.5) (layer F.Cu) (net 2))
 (segment (start 79.0448 33.3068) (end 77.8092 32.0712) (width 0.5) (layer F.Cu) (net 2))
 (segment (start 79.0448 36.9062) (end 79.0448 33.3068) (width 0.5) (layer F.Cu) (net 2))
 (segment (start 75.706 29.968) (end 77.8092 32.0712) (width 0.5) (layer F.Cu) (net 2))
 (segment (start 103.039399 40.378999) (end 104.5514 41.891) (width 0.5) (layer F.Cu) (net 13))
 (segment (start 103.039399 33.761397) (end 103.039399 40.378999) (width 0.5) (layer F.Cu) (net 13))
 (segment (start 99.246002 29.968) (end 103.039399 33.761397) (width 0.5) (layer F.Cu) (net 13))
 (segment (start 93.756 29.968) (end 99.246002 29.968) (width 0.5) (layer F.Cu) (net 13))
 (segment (start 39.606 47.018) (end 55.1558 47.018) (width 0.5) (layer F.Cu) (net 7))
 (segment (start 55.1558 47.018) (end 58.5115 50.3737) (width 0.5) (layer F.Cu) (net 7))
 (segment (start 58.5115 50.3737) (end 58.5896 50.3737) (width 0.5) (layer F.Cu) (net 7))
 (segment (start 58.5896 50.3737) (end 61.0071 52.7912) (width 0.5) (layer F.Cu) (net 7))
 (segment (start 61.0071 52.7912) (end 61.0071 53.0329) (width 0.5) (layer F.Cu) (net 7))
 (segment (start 61.0071 53.0329) (end 66.6176 58.6434) (width 0.5) (layer F.Cu) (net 7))
 (segment (start 66.6176 58.6434) (end 103.5238 58.6434) (width 0.5) (layer F.Cu) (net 7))
 (segment (start 103.5238 58.6434) (end 104.5514 59.671) (width 0.5) (layer F.Cu) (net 7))
 (segment (start 57.656 47.018) (end 61.5121 50.8741) (width 0.5) (layer F.Cu) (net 8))
 (segment (start 61.5121 50.8741) (end 63.4307 50.8741) (width 0.5) (layer F.Cu) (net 8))
 (segment (start 63.4307 50.8741) (end 69.6876 57.131) (width 0.5) (layer F.Cu) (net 8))
 (segment (start 69.6876 57.131) (end 104.5514 57.131) (width 0.5) (layer F.Cu) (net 8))
 (segment (start 100.8649 50.9045) (end 104.5514 54.591) (width 0.5) (layer F.Cu) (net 9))
 (segment (start 97.952498 50.9045) (end 100.8649 50.9045) (width 0.5) (layer F.Cu) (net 9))
 (segment (start 97.515997 50.467999) (end 97.952498 50.9045) (width 0.5) (layer F.Cu) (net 9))
 (segment (start 92.696001 50.467999) (end 97.515997 50.467999) (width 0.5) (layer F.Cu) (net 9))
 (segment (start 89.246002 47.018) (end 92.696001 50.467999) (width 0.5) (layer F.Cu) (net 9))
 (segment (start 75.706 47.018) (end 89.246002 47.018) (width 0.5) (layer F.Cu) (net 9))
 (segment (start 93.756 47.018) (end 99.5184 47.018) (width 0.5) (layer F.Cu) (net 10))
 (segment (start 99.5184 47.018) (end 104.5514 52.051) (width 0.5) (layer F.Cu) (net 10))
 (segment (start 93.756 64.068) (end 103.7133 64.068) (width 0.5) (layer F.Cu) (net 5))
 (segment (start 103.7133 64.068) (end 113.1903 54.591) (width 0.5) (layer F.Cu) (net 5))
 (segment (start 113.1903 54.591) (end 119.7714 54.591) (width 0.5) (layer F.Cu) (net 5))
 (segment (start 111.806 64.068) (end 118.743 57.131) (width 0.5) (layer B.Cu) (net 6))
 (segment (start 118.743 57.131) (end 119.7714 57.131) (width 0.5) (layer B.Cu) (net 6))
 (segment (start 107.063411 31.703091) (end 104.55132 29.191) (width 0.5) (layer B.Cu) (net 4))
 (segment (start 107.063411 60.810977) (end 107.063411 31.703091) (width 0.5) (layer B.Cu) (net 4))
 (segment (start 97.915999 67.918001) (end 99.956387 67.918001) (width 0.5) (layer B.Cu) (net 4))
 (segment (start 97.515997 67.517999) (end 97.915999 67.918001) (width 0.5) (layer B.Cu) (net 4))
 (segment (start 92.579999 67.517999) (end 97.515997 67.517999) (width 0.5) (layer B.Cu) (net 4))
 (segment (start 99.956387 67.918001) (end 107.063411 60.810977) (width 0.5) (layer B.Cu) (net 4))
 (segment (start 92.179997 67.918001) (end 92.579999 67.517999) (width 0.5) (layer B.Cu) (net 4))
 (segment (start 84.490306 67.918001) (end 92.179997 67.918001) (width 0.5) (layer B.Cu) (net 4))
 (segment (start 83.403149 66.830843) (end 84.490306 67.918001) (width 0.5) (layer B.Cu) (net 4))
 (segment (start 82.655138 66.830843) (end 83.403149 66.830843) (width 0.5) (layer B.Cu) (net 4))
 (segment (start 106.063401 60.396761) (end 106.063401 33.243001) (width 0.5) (layer B.Cu) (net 14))
 (segment (start 105.277161 61.183001) (end 106.063401 60.396761) (width 0.5) (layer B.Cu) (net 14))
 (segment (start 91.150997 61.183001) (end 105.277161 61.183001) (width 0.5) (layer B.Cu) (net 14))
 (segment (start 106.063401 33.243001) (end 104.5514 31.731) (width 0.5) (layer B.Cu) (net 14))
 (segment (start 85.834272 66.499726) (end 91.150997 61.183001) (width 0.5) (layer B.Cu) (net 14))
 (segment (start 84.486258 66.499726) (end 85.834272 66.499726) (width 0.5) (layer B.Cu) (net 14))
 (segment (start 83.198386 65.211854) (end 84.486258 66.499726) (width 0.5) (layer B.Cu) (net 14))
 (segment (start 82.235146 65.211854) (end 83.198386 65.211854) (width 0.5) (layer B.Cu) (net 14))
 (segment (start 81.676817 65.770183) (end 82.235146 65.211854) (width 0.5) (layer B.Cu) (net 14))
 (segment (start 81.594478 65.770183) (end 81.676817 65.770183) (width 0.5) (layer B.Cu) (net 14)))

